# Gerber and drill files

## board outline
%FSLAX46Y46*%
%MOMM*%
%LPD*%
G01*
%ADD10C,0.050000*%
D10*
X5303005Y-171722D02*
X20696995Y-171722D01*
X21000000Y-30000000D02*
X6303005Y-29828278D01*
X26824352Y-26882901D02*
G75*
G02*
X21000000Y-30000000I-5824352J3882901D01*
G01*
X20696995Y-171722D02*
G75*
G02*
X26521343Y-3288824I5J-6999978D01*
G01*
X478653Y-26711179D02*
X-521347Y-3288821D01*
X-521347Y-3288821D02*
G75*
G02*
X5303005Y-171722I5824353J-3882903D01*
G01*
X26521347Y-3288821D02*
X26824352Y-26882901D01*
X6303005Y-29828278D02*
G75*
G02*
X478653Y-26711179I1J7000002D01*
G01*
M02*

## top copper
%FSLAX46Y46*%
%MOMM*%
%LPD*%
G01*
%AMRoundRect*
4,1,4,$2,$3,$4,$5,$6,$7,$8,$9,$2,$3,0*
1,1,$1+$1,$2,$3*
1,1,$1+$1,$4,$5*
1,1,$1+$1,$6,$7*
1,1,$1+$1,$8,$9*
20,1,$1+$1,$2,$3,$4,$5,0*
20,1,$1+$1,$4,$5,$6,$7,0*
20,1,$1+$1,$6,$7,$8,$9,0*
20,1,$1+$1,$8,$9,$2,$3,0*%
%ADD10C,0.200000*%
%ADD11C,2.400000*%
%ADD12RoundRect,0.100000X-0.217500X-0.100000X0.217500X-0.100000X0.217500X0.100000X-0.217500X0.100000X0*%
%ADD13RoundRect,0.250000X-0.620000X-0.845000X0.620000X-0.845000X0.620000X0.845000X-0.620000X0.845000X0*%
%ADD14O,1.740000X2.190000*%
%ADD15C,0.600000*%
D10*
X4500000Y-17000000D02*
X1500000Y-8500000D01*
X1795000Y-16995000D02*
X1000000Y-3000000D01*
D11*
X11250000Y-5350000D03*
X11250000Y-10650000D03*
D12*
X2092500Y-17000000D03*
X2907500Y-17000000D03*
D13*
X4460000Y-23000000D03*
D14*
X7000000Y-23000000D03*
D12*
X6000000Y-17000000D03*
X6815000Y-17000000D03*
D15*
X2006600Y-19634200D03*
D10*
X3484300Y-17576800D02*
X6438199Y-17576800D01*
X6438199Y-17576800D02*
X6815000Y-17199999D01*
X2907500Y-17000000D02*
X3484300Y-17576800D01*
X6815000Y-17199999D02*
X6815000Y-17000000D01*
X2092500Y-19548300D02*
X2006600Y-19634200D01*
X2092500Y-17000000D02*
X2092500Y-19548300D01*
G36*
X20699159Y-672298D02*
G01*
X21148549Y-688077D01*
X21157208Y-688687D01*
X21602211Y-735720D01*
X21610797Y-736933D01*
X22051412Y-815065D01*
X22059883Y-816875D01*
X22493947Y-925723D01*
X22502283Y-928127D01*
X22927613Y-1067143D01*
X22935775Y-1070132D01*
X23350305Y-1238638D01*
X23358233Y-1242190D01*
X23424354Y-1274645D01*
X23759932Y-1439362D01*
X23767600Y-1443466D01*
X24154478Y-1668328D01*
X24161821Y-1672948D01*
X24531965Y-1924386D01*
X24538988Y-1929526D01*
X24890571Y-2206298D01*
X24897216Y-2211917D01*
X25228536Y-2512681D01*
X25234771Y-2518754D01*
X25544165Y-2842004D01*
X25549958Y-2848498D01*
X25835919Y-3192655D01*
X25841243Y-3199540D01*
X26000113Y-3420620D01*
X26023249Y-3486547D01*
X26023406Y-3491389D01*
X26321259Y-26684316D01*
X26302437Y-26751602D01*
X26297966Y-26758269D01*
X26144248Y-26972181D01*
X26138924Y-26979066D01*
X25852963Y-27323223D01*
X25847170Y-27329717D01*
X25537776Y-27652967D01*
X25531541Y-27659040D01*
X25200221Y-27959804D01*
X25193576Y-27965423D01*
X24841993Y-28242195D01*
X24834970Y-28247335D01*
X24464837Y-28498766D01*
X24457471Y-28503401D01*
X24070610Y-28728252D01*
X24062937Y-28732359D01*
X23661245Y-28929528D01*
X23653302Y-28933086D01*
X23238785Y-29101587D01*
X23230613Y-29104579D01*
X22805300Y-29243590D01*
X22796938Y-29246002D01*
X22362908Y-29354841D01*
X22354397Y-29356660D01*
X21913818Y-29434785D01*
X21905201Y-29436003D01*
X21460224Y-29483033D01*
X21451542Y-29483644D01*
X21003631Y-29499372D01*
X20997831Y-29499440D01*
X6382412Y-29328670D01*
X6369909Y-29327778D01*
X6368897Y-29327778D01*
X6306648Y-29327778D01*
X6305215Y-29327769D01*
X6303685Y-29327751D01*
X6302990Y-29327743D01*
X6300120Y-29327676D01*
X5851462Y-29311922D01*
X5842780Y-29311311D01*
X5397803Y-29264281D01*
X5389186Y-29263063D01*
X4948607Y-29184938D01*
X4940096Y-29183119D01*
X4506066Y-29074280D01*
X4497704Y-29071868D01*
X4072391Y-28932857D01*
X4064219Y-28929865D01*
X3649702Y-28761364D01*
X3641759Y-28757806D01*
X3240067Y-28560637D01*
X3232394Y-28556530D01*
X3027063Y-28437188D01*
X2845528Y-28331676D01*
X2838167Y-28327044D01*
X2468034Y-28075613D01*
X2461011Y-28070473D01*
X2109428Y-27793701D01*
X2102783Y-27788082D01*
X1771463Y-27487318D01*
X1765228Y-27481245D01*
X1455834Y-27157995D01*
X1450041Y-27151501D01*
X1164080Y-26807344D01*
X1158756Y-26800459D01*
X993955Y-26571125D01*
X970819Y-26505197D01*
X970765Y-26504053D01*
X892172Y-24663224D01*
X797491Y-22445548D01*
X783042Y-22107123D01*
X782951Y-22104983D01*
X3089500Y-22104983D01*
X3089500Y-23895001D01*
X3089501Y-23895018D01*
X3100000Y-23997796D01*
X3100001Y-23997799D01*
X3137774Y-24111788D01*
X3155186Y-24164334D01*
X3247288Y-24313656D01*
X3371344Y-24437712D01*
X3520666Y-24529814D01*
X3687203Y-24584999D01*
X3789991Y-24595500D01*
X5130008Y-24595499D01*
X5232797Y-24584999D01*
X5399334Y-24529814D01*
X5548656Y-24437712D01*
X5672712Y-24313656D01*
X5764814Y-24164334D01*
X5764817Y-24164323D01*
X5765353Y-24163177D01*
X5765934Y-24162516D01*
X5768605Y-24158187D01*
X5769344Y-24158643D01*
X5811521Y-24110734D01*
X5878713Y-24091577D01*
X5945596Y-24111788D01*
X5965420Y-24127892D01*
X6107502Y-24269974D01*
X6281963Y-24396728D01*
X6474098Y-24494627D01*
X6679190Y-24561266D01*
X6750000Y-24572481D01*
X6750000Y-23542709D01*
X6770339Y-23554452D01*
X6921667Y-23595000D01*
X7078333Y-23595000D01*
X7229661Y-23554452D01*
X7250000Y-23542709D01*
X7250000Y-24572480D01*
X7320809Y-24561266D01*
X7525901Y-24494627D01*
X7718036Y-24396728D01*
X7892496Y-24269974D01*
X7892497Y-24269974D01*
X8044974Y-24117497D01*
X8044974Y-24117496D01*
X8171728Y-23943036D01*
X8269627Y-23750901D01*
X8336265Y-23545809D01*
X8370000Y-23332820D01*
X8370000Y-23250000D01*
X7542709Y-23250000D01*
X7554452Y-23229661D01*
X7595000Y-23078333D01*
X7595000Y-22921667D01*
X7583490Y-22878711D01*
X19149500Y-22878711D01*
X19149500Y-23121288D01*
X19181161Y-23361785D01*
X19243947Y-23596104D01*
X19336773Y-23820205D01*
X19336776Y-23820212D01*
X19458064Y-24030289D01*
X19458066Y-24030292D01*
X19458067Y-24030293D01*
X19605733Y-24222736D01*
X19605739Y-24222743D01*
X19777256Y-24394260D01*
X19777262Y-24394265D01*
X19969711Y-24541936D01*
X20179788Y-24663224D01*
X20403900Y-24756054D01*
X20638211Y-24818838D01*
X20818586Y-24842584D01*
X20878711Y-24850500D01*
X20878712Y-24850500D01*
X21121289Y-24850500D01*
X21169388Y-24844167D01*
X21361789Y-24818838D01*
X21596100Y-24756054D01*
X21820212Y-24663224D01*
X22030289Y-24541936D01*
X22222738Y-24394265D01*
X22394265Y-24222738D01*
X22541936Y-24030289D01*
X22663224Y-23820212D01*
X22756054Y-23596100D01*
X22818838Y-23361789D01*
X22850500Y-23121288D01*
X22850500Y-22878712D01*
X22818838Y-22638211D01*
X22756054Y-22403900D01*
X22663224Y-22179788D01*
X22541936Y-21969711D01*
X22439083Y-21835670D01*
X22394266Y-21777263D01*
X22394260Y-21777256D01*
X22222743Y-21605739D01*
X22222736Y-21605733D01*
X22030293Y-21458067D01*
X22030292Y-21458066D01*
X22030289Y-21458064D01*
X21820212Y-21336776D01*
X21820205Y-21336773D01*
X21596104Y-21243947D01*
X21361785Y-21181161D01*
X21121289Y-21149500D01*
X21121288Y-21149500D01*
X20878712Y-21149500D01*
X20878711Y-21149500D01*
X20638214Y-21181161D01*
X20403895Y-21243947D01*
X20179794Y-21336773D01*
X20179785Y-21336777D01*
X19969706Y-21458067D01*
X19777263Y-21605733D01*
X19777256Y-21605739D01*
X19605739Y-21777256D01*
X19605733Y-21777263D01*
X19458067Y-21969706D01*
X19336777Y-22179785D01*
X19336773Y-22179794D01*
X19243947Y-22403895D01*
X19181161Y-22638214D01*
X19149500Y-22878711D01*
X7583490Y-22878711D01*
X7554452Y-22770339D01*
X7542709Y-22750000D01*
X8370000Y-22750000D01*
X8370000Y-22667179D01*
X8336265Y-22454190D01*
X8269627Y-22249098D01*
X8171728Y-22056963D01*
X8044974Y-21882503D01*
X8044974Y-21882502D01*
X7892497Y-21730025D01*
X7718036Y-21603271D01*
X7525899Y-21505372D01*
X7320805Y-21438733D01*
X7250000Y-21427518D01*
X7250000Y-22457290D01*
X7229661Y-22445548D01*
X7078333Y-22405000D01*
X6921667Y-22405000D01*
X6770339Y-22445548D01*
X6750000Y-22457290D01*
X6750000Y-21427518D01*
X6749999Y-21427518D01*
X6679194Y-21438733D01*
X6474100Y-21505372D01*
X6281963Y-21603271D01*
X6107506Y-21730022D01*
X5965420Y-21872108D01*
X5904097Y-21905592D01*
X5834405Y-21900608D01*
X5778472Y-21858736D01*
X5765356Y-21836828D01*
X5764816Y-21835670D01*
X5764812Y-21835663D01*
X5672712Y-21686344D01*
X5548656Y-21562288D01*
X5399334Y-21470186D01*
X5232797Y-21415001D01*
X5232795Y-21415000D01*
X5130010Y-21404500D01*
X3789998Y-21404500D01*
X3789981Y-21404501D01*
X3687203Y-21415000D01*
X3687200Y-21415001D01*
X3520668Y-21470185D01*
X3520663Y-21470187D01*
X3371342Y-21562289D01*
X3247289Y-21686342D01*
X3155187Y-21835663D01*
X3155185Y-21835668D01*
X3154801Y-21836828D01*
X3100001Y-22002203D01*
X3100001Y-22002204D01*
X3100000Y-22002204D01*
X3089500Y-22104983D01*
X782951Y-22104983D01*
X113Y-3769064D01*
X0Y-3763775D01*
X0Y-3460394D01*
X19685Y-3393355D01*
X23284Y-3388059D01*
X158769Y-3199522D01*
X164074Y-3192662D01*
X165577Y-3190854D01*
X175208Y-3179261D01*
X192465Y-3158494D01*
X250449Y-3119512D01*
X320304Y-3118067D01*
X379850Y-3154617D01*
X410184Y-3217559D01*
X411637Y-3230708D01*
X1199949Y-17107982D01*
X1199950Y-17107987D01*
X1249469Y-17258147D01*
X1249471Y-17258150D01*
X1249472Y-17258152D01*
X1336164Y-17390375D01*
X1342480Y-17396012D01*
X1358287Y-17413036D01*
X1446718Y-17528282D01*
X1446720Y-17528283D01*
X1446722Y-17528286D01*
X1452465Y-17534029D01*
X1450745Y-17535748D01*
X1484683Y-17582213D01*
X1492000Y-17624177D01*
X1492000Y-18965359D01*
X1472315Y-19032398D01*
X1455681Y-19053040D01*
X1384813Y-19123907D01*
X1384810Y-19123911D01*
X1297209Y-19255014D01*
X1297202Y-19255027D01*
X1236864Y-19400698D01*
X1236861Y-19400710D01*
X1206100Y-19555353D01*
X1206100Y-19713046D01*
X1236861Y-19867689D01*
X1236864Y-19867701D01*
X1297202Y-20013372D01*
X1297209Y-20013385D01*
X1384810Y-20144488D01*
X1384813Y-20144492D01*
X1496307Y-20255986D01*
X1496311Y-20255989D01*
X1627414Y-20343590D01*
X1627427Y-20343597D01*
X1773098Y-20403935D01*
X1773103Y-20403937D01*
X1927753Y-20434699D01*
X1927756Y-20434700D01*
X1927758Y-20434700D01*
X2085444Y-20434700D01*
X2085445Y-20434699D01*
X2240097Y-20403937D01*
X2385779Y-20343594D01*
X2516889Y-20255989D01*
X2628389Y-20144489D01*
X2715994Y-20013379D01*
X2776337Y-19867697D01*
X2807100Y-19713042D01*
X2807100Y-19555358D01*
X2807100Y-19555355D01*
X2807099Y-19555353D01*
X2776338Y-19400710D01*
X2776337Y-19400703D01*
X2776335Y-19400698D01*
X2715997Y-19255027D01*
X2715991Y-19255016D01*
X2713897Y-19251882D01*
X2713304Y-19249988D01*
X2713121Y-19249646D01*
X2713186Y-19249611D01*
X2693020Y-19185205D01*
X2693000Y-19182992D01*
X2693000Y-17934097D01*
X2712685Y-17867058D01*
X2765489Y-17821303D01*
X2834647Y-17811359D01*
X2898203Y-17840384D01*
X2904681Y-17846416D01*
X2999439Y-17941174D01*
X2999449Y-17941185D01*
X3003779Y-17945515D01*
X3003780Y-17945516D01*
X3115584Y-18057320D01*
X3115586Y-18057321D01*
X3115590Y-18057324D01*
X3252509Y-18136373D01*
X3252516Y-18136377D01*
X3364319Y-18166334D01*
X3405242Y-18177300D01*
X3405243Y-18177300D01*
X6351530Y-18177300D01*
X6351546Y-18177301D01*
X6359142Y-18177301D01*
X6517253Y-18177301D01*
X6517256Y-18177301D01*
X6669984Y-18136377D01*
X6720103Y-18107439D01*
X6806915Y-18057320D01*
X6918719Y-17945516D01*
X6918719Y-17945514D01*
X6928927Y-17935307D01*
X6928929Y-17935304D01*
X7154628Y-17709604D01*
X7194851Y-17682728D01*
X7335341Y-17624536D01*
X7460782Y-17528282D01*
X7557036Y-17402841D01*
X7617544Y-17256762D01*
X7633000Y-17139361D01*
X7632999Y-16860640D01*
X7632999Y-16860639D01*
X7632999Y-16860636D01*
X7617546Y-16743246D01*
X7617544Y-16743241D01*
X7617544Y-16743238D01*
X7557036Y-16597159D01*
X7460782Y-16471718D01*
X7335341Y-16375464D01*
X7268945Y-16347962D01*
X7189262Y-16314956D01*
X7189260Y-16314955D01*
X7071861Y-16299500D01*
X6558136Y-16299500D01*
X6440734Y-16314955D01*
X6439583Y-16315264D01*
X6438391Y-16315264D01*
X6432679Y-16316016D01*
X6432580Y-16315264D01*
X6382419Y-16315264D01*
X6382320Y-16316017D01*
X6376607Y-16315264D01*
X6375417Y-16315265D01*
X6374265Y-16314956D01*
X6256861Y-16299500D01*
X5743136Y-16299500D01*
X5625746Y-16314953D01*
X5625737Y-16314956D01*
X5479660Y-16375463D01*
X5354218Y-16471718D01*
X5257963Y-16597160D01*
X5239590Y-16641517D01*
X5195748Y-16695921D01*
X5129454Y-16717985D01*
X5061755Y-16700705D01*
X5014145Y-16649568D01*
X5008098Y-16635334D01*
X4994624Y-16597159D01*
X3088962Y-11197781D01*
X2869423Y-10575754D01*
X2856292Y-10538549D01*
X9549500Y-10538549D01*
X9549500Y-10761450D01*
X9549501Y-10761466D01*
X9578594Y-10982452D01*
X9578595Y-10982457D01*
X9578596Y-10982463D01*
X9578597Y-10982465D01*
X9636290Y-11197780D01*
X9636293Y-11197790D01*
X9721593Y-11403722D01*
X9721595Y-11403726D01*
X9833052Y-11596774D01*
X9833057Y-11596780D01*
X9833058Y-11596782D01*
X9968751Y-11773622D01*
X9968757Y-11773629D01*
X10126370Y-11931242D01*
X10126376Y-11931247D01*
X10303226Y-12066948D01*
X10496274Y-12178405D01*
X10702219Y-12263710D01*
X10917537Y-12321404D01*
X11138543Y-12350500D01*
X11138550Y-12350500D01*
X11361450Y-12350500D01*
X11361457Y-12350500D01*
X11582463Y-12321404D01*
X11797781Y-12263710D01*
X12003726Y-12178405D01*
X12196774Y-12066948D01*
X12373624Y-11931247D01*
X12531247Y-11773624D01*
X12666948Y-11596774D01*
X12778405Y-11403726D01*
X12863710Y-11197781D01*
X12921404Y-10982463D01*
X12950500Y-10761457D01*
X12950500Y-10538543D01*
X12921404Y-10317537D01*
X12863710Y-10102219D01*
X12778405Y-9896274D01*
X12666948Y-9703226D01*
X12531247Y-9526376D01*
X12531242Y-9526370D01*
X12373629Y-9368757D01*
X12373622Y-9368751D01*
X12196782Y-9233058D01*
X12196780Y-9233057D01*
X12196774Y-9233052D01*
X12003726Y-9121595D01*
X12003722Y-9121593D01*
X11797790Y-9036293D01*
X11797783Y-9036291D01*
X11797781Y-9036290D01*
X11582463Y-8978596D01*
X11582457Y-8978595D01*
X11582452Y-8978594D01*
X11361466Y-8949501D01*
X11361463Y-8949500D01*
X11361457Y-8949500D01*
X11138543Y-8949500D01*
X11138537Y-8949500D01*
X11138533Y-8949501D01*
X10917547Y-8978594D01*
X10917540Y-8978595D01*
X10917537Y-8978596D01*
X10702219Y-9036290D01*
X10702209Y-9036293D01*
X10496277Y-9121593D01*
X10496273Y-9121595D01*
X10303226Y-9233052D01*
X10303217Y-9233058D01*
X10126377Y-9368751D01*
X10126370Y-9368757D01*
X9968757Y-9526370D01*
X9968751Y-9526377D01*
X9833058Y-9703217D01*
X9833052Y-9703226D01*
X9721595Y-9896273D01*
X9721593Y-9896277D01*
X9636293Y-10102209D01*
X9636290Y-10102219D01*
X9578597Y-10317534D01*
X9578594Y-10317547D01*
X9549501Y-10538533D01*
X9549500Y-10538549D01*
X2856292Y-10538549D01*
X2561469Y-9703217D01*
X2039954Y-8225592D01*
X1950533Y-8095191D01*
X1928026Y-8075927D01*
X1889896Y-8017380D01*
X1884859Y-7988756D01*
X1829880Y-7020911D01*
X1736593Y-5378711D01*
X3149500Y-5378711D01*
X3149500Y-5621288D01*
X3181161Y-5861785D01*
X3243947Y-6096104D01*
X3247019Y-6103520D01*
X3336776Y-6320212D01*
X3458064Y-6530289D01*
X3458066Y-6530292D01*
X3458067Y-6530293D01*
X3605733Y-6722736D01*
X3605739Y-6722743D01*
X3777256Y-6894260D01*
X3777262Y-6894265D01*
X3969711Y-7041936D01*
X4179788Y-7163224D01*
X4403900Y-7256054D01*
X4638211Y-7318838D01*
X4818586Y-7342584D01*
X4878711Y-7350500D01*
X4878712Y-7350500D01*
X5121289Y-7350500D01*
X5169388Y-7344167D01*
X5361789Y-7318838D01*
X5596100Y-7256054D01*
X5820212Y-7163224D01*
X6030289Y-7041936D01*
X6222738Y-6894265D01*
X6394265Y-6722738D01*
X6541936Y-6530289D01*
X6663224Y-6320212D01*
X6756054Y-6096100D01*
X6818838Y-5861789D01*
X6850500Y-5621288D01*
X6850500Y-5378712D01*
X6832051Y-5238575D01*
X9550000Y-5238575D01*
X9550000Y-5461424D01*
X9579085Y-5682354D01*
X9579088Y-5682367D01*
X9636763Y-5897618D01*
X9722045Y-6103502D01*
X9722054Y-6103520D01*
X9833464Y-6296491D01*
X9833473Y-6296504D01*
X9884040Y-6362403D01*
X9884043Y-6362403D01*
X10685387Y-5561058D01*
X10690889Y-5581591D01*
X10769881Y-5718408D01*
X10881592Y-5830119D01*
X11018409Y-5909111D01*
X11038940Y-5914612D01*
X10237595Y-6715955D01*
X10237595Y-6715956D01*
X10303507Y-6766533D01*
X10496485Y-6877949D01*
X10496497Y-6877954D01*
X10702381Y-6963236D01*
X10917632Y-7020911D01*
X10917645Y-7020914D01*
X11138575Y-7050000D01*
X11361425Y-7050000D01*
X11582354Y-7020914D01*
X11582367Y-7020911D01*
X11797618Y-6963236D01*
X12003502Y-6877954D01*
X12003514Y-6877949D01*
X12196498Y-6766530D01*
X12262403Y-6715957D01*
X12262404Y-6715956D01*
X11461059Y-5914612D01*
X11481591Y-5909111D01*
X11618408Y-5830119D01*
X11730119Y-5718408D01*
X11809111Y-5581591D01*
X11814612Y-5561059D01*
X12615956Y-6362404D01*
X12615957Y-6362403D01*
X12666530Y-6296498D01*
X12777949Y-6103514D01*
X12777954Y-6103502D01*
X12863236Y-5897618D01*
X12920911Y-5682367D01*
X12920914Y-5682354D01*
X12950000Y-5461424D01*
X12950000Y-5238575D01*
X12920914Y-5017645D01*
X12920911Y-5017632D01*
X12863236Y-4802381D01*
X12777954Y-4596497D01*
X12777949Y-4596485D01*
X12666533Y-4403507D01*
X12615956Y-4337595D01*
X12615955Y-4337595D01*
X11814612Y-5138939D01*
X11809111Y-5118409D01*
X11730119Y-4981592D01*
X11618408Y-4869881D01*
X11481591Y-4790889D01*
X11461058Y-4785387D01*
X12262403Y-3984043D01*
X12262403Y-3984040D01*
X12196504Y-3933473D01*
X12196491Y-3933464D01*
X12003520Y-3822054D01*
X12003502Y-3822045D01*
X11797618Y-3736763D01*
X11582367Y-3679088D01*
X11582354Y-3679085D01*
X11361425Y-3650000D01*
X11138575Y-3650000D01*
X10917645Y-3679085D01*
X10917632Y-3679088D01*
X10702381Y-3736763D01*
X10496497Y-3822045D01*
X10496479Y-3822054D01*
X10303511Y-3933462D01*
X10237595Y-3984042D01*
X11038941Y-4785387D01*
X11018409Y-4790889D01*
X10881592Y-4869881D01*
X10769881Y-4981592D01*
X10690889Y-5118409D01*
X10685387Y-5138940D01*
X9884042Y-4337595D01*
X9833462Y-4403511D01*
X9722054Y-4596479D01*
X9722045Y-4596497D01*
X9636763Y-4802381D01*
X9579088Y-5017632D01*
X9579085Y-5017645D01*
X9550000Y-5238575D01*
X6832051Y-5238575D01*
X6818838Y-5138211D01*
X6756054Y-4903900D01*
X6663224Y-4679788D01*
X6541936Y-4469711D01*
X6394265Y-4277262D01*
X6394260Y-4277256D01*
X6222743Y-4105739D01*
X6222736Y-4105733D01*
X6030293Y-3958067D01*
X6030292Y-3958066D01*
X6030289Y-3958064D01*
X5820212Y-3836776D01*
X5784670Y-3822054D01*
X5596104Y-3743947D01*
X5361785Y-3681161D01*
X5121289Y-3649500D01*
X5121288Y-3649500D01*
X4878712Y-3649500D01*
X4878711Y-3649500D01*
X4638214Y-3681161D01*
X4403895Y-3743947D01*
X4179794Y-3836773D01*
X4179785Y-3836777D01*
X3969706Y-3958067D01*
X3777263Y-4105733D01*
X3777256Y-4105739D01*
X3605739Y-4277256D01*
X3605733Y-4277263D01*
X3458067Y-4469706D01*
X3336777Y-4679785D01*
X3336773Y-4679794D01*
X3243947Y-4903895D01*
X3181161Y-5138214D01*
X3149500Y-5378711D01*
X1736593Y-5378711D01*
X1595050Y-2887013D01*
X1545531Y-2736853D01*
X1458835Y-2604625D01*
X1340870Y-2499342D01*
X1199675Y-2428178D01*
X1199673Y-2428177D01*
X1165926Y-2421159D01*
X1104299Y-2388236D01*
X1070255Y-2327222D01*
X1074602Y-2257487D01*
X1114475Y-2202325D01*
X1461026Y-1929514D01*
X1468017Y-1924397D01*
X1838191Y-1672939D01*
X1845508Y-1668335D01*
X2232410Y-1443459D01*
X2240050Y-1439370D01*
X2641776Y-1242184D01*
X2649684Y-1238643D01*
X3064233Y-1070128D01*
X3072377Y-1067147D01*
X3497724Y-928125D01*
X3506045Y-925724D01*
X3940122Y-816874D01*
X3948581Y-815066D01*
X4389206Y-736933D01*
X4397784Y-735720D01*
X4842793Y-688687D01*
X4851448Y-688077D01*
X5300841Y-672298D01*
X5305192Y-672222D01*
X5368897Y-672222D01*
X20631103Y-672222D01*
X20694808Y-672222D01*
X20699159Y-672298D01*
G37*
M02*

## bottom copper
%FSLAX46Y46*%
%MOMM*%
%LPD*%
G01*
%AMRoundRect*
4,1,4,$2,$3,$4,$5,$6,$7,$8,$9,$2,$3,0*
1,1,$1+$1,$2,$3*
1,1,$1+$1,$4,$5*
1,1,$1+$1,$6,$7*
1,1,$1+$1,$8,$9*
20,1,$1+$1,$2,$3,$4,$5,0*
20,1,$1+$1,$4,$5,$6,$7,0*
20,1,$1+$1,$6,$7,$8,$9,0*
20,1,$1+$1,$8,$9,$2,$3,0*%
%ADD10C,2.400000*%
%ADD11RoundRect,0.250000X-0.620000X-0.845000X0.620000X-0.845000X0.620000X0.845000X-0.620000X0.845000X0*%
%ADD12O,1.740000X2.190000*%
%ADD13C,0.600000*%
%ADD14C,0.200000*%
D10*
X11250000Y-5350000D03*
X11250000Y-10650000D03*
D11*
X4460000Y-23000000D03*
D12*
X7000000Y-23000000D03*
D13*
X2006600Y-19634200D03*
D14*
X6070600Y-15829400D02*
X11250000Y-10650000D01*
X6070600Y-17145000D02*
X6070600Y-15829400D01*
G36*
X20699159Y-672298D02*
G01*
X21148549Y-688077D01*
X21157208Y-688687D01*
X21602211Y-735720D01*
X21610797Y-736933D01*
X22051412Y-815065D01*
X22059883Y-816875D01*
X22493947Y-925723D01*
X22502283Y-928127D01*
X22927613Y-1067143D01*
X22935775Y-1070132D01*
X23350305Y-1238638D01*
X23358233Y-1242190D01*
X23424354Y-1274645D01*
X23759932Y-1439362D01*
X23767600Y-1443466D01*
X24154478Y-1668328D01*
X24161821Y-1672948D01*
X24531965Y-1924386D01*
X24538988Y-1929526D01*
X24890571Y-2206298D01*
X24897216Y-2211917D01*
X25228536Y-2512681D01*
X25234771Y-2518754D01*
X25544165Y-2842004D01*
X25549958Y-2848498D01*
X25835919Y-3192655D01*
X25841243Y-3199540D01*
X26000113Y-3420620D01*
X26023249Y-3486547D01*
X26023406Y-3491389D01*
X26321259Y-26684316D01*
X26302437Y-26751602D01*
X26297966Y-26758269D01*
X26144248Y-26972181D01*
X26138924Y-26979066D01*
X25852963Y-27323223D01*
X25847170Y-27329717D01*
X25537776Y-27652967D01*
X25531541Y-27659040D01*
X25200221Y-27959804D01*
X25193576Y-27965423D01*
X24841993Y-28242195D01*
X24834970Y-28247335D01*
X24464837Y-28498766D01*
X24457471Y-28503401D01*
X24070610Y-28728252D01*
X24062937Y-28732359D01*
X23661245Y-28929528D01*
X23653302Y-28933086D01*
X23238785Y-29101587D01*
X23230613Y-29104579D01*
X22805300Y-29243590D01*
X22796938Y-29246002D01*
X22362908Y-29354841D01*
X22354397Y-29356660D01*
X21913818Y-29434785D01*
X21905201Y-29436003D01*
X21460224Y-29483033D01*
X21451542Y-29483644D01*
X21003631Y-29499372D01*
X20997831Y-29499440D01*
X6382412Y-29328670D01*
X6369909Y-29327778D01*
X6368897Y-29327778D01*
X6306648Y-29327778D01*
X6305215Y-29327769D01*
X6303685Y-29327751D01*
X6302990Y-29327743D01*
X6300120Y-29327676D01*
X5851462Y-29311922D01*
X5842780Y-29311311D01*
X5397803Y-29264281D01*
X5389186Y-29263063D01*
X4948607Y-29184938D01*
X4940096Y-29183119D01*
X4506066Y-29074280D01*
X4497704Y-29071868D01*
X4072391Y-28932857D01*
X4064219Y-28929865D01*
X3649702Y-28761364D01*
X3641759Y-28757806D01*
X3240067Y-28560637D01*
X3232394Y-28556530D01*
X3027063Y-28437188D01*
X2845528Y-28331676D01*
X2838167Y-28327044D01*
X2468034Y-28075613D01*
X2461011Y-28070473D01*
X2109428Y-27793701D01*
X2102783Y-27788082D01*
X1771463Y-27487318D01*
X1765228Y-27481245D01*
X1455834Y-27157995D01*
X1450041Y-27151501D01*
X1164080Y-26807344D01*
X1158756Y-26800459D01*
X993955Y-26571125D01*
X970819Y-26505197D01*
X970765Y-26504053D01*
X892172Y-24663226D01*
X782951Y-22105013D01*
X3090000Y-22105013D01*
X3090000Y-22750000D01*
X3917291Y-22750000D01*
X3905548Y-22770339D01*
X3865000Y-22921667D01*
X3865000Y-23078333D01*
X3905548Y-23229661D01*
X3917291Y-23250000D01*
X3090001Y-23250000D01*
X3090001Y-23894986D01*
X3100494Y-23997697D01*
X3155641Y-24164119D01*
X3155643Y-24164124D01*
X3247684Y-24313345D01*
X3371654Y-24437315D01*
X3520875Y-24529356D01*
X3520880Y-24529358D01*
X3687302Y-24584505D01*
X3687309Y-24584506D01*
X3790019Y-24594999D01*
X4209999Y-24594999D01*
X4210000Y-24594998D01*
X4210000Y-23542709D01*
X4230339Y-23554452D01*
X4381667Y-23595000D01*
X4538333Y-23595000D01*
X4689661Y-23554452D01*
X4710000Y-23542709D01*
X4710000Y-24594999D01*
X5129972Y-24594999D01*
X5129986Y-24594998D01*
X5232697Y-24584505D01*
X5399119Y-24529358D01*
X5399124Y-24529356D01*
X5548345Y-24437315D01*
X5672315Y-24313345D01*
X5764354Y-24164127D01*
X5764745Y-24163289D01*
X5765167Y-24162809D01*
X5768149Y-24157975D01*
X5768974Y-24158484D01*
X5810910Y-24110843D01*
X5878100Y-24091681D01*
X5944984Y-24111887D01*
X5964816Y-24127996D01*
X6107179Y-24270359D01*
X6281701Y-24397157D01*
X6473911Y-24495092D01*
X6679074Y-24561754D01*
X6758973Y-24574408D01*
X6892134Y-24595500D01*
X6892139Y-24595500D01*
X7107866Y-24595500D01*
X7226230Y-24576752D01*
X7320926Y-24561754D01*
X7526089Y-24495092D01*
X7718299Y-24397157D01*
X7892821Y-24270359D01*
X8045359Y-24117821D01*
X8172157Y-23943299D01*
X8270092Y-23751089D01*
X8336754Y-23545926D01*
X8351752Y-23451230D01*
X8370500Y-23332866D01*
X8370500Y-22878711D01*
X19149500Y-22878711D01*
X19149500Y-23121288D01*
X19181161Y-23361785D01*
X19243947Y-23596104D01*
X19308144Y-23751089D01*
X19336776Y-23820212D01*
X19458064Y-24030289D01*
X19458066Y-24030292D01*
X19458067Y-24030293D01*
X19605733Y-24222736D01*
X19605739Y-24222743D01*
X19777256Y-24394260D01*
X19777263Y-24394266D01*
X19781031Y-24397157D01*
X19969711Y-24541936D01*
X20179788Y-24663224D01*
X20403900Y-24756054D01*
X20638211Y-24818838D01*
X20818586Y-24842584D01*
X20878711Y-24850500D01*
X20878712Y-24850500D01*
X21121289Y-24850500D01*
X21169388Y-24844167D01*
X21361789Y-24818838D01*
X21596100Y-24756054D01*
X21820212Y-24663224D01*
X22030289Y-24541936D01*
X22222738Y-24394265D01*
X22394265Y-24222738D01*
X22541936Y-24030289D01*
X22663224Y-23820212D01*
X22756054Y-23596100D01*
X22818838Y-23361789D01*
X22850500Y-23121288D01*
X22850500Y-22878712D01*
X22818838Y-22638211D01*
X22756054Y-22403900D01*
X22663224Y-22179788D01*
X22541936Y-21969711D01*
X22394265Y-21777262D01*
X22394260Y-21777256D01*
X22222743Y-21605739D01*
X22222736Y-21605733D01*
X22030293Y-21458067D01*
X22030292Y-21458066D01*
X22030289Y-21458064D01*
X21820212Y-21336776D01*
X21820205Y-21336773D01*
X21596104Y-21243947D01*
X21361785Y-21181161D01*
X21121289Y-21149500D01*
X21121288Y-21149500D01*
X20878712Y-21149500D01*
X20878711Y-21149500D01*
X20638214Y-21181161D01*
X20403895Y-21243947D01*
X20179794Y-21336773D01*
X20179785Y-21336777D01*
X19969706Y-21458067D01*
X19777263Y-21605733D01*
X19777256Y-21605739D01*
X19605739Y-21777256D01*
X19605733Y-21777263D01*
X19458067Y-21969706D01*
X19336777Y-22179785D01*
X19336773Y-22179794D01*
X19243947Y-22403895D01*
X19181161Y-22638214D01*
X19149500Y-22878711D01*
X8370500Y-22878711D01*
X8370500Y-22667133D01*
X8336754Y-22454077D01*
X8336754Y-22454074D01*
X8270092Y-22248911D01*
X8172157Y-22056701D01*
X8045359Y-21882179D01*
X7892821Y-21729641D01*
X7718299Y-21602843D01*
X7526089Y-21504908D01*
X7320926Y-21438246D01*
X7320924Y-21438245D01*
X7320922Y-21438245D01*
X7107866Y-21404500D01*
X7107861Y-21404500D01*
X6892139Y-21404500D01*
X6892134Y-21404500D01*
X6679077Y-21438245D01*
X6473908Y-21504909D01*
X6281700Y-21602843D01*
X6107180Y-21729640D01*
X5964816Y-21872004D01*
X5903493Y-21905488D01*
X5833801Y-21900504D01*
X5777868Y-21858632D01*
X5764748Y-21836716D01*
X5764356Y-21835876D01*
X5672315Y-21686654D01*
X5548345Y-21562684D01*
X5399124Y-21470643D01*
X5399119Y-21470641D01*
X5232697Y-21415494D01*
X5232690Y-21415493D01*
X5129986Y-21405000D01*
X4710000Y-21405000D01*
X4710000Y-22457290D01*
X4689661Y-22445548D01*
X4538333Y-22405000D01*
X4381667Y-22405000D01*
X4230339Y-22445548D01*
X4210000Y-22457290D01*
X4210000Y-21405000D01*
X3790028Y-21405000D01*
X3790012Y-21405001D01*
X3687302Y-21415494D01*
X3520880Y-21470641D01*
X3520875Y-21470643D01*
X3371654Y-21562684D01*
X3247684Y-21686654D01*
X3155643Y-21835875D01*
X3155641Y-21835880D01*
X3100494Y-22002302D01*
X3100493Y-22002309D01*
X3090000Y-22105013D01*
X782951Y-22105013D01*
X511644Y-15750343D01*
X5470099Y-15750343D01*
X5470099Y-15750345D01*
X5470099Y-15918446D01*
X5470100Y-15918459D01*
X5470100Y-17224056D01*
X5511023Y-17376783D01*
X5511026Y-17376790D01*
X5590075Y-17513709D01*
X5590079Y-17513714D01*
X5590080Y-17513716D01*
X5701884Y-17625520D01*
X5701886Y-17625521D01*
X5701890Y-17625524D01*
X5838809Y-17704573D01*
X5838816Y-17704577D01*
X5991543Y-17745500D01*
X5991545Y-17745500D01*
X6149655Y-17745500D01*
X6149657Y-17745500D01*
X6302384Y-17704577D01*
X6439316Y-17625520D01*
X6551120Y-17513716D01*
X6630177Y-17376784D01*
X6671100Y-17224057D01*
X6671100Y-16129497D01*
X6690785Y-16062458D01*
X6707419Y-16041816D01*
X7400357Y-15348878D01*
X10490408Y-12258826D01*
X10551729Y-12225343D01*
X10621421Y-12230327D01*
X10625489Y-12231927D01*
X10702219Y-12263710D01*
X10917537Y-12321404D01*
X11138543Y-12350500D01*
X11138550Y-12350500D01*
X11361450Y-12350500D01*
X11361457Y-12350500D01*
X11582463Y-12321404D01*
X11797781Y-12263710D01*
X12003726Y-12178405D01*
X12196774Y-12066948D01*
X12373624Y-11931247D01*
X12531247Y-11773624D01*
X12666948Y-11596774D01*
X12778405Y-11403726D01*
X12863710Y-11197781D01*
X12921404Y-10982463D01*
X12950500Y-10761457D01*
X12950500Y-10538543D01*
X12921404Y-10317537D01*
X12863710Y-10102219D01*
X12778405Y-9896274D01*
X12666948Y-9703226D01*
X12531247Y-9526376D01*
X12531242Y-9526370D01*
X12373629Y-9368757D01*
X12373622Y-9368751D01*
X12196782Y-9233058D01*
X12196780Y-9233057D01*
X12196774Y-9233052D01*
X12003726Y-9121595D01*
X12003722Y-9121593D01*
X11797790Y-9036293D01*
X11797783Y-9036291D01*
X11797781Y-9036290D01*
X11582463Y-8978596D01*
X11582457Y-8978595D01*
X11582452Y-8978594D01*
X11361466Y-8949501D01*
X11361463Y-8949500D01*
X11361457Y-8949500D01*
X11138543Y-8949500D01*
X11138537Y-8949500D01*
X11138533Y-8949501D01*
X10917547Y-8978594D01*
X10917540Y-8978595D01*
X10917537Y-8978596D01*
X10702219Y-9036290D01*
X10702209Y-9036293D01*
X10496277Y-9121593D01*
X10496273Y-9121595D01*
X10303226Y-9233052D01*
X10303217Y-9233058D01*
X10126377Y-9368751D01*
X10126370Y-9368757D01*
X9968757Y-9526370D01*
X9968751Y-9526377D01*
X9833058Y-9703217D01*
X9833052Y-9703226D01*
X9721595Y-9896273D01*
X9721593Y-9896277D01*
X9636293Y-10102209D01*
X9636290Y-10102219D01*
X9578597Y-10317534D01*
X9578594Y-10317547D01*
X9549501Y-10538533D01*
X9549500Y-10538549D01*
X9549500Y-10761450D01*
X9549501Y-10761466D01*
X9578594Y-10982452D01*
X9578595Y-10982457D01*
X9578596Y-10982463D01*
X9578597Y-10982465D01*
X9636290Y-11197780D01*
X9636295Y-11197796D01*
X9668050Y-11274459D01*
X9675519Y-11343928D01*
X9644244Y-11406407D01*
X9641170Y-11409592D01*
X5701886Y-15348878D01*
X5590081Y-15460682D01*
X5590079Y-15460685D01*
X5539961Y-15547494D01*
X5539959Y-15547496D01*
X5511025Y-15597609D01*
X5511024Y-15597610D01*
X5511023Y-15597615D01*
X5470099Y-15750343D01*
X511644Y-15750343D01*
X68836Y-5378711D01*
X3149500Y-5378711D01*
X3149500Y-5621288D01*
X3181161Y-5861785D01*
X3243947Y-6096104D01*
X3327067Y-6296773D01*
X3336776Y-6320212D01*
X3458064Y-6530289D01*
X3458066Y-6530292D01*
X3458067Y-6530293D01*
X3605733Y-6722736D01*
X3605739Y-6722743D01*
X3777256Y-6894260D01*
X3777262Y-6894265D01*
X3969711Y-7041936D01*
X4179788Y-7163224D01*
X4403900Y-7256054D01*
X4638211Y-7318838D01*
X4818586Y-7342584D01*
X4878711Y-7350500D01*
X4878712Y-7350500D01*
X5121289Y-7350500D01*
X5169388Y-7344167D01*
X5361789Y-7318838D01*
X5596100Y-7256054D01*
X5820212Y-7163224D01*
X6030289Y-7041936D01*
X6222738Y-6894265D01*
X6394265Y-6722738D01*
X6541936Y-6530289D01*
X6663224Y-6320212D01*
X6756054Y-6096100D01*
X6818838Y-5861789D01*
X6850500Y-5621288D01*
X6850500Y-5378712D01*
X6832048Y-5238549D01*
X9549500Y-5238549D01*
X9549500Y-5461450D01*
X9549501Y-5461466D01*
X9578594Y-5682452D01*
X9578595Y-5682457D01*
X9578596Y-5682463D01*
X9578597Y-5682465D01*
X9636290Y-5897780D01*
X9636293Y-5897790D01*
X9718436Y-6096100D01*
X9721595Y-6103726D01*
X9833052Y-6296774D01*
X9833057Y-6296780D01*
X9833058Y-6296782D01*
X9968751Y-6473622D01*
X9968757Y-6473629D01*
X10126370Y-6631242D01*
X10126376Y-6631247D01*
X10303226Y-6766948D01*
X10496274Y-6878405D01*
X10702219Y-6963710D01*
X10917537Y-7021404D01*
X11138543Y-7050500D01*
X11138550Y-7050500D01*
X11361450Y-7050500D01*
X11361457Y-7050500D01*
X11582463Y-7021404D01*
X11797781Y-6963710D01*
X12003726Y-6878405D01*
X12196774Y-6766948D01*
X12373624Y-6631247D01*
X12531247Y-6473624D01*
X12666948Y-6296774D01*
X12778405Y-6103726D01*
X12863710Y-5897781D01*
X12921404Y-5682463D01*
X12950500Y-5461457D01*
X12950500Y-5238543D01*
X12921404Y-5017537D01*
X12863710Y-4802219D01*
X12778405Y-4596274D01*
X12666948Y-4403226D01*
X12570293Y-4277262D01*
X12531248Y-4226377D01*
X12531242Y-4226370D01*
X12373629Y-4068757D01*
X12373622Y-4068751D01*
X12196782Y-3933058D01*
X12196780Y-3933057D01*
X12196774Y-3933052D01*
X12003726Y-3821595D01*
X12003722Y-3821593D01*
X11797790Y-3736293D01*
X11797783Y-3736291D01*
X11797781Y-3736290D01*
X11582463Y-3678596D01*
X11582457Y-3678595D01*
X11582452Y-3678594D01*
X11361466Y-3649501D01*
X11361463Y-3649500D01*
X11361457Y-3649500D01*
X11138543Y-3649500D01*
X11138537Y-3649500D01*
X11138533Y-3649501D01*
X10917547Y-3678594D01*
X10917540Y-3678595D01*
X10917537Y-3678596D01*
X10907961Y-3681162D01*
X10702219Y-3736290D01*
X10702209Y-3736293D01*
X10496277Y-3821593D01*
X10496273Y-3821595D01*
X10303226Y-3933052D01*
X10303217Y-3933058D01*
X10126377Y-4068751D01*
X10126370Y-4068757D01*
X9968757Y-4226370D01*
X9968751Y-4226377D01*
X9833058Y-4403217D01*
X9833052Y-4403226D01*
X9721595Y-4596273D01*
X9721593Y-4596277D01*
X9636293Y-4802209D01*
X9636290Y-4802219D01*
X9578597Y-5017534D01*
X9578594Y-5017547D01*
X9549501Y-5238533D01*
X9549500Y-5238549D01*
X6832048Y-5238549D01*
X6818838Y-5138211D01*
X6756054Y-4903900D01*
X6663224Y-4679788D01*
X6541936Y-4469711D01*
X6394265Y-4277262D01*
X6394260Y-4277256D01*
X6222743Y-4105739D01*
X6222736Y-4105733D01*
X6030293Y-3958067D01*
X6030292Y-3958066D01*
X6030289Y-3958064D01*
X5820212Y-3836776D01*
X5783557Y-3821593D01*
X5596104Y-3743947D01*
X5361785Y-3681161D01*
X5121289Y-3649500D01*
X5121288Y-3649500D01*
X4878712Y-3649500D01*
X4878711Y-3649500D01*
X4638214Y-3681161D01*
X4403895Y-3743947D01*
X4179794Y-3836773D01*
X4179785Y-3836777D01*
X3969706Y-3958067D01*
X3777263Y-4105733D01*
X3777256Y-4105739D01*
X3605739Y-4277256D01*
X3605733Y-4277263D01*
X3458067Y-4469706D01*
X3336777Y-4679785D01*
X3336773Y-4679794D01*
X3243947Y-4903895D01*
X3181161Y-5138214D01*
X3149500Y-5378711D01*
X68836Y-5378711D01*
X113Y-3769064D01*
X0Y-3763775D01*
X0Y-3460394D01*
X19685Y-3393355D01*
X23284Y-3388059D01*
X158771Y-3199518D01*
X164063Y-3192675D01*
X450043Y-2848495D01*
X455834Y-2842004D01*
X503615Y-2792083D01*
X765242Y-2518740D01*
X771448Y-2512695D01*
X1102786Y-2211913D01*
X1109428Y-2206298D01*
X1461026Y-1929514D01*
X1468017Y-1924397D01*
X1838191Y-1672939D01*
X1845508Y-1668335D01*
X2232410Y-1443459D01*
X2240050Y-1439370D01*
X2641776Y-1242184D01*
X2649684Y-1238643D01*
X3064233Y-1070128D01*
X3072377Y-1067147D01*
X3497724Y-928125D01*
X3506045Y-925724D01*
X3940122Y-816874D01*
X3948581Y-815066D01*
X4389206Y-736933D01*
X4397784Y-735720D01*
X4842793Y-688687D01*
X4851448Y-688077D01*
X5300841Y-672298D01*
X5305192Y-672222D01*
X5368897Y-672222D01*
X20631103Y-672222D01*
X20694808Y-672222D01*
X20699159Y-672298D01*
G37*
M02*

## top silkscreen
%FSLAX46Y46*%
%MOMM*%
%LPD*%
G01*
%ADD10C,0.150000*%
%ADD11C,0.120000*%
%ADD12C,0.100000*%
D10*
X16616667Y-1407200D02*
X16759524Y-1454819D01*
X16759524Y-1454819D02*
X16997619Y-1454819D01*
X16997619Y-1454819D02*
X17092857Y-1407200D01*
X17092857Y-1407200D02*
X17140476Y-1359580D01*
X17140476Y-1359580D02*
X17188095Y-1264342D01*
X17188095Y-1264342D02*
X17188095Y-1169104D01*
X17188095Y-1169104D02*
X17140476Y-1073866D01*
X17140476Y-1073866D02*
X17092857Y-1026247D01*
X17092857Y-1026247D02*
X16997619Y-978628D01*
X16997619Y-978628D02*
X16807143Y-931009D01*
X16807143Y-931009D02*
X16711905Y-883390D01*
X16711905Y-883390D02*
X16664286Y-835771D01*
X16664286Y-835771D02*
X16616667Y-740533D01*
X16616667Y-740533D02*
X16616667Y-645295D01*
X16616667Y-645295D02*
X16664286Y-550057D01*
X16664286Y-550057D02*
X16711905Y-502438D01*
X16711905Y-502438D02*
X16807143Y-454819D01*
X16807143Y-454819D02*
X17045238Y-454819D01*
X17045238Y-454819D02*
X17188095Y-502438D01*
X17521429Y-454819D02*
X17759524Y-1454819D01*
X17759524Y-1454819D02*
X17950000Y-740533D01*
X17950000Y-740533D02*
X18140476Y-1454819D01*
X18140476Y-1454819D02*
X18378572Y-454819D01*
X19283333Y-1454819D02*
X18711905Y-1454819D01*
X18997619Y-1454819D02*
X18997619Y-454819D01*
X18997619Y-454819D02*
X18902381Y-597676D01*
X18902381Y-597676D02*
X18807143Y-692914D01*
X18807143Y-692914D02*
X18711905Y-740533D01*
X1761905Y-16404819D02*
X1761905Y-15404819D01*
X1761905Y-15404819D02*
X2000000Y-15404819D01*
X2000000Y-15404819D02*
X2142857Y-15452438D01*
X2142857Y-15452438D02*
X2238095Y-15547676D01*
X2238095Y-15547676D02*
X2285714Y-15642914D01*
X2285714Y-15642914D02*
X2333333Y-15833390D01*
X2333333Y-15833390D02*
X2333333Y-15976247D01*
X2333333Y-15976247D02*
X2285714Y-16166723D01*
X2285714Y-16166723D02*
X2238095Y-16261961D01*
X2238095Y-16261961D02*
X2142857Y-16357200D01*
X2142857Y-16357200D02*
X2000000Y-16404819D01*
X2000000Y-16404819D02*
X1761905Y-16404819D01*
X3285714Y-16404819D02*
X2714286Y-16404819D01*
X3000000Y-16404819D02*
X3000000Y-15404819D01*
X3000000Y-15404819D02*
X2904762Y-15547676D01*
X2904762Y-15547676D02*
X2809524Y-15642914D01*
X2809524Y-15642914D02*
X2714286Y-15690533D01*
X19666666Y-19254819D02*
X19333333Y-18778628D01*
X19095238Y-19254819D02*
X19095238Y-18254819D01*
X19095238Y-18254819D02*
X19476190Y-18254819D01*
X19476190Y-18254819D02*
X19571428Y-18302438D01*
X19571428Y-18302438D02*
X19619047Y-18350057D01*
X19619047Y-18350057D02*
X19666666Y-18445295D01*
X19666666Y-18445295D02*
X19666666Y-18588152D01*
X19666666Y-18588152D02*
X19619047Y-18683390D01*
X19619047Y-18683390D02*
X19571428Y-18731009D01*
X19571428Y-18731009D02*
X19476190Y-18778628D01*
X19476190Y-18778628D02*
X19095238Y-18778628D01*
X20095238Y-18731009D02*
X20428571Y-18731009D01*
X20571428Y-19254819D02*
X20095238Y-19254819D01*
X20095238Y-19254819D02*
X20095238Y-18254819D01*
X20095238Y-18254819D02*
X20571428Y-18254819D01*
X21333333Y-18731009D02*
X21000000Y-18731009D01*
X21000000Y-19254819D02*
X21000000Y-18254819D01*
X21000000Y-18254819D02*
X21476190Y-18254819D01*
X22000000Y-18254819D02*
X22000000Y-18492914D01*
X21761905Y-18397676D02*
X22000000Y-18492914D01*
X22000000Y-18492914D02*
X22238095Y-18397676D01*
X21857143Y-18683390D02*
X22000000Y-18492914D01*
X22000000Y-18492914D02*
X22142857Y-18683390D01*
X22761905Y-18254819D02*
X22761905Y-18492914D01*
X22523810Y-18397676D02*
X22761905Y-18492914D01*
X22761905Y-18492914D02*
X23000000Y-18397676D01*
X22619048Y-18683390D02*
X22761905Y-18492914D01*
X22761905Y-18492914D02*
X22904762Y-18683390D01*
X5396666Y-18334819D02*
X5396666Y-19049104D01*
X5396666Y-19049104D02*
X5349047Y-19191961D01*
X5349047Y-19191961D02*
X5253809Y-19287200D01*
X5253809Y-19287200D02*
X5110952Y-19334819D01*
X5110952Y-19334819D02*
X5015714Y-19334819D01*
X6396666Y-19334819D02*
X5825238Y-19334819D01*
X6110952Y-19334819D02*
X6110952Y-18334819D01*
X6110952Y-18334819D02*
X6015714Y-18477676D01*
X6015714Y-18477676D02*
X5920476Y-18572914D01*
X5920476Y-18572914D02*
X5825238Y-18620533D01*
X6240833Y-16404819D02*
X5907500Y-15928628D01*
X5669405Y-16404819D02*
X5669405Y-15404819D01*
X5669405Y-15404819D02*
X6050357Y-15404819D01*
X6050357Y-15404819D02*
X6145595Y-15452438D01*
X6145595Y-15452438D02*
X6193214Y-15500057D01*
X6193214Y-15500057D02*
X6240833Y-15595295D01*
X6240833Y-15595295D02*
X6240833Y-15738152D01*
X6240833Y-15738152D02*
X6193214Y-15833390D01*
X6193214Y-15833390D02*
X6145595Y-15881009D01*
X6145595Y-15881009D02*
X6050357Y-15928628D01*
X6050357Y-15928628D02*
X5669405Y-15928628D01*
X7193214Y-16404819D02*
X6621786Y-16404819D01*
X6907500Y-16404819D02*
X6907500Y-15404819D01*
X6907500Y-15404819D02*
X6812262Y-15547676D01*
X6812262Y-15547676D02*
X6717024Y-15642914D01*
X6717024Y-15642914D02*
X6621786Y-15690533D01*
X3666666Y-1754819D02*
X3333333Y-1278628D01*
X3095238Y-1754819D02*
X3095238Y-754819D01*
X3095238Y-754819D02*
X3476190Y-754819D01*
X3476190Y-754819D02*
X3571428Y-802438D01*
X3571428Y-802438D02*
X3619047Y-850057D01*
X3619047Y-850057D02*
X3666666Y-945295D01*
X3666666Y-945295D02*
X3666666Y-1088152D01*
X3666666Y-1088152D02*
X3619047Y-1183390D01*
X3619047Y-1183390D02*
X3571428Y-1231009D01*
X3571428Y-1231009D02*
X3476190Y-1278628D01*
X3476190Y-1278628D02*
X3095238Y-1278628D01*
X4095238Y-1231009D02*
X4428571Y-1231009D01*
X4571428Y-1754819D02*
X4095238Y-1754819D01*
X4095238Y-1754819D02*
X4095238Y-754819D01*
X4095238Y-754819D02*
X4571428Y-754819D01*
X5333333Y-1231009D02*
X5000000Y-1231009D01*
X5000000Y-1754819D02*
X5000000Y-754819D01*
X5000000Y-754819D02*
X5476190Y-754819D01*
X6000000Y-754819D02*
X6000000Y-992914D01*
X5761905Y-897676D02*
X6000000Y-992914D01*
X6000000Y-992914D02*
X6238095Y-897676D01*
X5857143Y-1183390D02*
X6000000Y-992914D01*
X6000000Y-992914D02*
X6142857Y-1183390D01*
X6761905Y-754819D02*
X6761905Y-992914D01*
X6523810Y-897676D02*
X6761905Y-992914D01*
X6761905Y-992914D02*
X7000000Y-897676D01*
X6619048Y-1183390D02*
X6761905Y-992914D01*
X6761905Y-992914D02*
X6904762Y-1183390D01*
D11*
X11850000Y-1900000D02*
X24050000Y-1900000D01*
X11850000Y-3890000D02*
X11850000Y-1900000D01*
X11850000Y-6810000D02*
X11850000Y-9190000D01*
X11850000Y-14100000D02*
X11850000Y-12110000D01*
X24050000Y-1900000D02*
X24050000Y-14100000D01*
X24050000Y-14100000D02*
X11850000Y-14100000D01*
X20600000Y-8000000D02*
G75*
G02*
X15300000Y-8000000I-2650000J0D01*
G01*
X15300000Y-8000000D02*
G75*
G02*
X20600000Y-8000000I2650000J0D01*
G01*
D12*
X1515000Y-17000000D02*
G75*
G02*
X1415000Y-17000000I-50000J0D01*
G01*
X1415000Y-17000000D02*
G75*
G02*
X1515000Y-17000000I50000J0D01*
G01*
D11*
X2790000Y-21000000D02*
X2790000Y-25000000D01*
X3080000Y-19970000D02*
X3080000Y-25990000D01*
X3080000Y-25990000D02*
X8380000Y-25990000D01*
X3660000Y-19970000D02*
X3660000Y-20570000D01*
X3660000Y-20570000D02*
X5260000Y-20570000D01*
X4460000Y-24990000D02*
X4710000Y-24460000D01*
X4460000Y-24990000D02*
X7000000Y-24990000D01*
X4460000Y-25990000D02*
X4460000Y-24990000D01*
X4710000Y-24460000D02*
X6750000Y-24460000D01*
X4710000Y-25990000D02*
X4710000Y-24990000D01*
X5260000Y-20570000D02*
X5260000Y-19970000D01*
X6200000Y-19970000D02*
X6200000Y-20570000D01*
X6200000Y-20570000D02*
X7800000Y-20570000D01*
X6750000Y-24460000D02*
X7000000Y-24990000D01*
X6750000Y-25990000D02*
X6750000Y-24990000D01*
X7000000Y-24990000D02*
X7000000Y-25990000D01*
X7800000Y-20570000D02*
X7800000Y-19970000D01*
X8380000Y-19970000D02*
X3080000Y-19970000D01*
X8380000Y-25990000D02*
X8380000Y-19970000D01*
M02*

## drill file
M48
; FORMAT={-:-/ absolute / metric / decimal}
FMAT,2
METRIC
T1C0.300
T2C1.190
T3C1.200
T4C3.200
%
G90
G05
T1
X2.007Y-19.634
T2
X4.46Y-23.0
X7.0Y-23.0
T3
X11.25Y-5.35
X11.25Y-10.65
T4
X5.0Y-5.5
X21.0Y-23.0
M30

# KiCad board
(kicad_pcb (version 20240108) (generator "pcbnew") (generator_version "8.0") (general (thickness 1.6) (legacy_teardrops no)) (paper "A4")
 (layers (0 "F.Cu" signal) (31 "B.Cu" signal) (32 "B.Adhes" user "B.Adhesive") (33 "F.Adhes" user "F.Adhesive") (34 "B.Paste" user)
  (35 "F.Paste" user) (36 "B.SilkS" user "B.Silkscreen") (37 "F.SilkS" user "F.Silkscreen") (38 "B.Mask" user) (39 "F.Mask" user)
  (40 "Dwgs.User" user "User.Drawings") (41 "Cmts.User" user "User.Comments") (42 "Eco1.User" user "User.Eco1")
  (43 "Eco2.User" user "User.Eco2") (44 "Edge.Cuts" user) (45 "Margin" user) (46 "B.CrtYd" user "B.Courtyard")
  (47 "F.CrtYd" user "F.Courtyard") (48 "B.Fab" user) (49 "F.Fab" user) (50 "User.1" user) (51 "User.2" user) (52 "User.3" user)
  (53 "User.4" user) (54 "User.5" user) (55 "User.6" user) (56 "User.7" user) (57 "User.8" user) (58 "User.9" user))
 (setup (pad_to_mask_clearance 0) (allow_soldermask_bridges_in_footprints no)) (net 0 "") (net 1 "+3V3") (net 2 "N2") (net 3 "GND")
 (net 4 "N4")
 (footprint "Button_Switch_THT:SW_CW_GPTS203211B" (layer "F.Cu") (at 11.25 5.35)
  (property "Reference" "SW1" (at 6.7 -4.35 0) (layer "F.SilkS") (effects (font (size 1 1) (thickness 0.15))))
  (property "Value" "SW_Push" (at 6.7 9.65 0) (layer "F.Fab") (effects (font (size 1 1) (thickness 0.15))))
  (fp_line (start 0.6 -3.45) (end 12.8 -3.45) (stroke (width 0.12) (type solid)) (layer "F.SilkS"))
  (fp_line (start 0.6 -1.46) (end 0.6 -3.45) (stroke (width 0.12) (type solid)) (layer "F.SilkS"))
  (fp_line (start 0.6 1.46) (end 0.6 3.84) (stroke (width 0.12) (type solid)) (layer "F.SilkS"))
  (fp_line (start 0.6 8.75) (end 0.6 6.76) (stroke (width 0.12) (type solid)) (layer "F.SilkS"))
  (fp_line (start 12.8 -3.45) (end 12.8 8.75) (stroke (width 0.12) (type solid)) (layer "F.SilkS"))
  (fp_line (start 12.8 8.75) (end 0.6 8.75) (stroke (width 0.12) (type solid)) (layer "F.SilkS"))
  (fp_circle (center 6.7 2.65) (end 9.35 2.65) (stroke (width 0.12) (type solid)) (fill none) (layer "F.SilkS"))
  (pad "1" thru_hole circle (at 0 0) (size 2.4 2.4) (drill 1.2) (layers "*.Cu" "*.Mask") (remove_unused_layers no) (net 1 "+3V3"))
  (pad "2" thru_hole circle (at 0 5.3) (size 2.4 2.4) (drill 1.2) (layers "*.Cu" "*.Mask") (remove_unused_layers no) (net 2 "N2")))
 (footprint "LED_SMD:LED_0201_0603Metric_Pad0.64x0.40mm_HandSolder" (layer "F.Cu") (at 2.5 17)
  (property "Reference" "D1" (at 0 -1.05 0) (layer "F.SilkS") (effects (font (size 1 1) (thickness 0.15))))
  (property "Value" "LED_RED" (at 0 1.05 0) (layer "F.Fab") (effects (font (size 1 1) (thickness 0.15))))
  (fp_circle (center -1.035 0) (end -0.985 0) (stroke (width 0.1) (type solid)) (fill none) (layer "F.SilkS"))
  (pad "" smd roundrect (at -0.4325 0) (size 0.458 0.36) (layers "F.Paste") (roundrect_rratio 0.25))
  (pad "" smd roundrect (at 0.4325 0) (size 0.458 0.36) (layers "F.Paste") (roundrect_rratio 0.25))
  (pad "1" smd roundrect (at -0.4075 0) (size 0.635 0.4) (layers "F.Cu" "F.Mask") (roundrect_rratio 0.25) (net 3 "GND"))
  (pad "2" smd roundrect (at 0.4075 0) (size 0.635 0.4) (layers "F.Cu" "F.Mask") (roundrect_rratio 0.25) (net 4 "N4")))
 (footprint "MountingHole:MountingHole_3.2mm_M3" (layer "F.Cu") (at 21 23)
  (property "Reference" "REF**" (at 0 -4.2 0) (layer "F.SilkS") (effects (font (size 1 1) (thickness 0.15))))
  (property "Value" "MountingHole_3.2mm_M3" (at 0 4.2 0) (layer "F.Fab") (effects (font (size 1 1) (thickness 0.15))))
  (pad "" np_thru_hole circle (at 0 0) (size 3.2 3.2) (drill 3.2) (layers "*.Cu" "*.Mask")))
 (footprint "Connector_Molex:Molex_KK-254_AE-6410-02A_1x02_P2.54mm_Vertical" (layer "F.Cu") (at 4.46 23)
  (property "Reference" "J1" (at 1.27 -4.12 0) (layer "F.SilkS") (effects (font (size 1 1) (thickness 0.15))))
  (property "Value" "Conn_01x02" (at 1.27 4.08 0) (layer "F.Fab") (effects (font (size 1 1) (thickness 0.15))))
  (fp_line (start -1.67 -2) (end -1.67 2) (stroke (width 0.12) (type solid)) (layer "F.SilkS"))
  (fp_line (start -1.38 -3.03) (end -1.38 2.99) (stroke (width 0.12) (type solid)) (layer "F.SilkS"))
  (fp_line (start -1.38 2.99) (end 3.92 2.99) (stroke (width 0.12) (type solid)) (layer "F.SilkS"))
  (fp_line (start -0.8 -3.03) (end -0.8 -2.43) (stroke (width 0.12) (type solid)) (layer "F.SilkS"))
  (fp_line (start -0.8 -2.43) (end 0.8 -2.43) (stroke (width 0.12) (type solid)) (layer "F.SilkS"))
  (fp_line (start 0 1.99) (end 0.25 1.46) (stroke (width 0.12) (type solid)) (layer "F.SilkS"))
  (fp_line (start 0 1.99) (end 2.54 1.99) (stroke (width 0.12) (type solid)) (layer "F.SilkS"))
  (fp_line (start 0 2.99) (end 0 1.99) (stroke (width 0.12) (type solid)) (layer "F.SilkS"))
  (fp_line (start 0.25 1.46) (end 2.29 1.46) (stroke (width 0.12) (type solid)) (layer "F.SilkS"))
  (fp_line (start 0.25 2.99) (end 0.25 1.99) (stroke (width 0.12) (type solid)) (layer "F.SilkS"))
  (fp_line (start 0.8 -2.43) (end 0.8 -3.03) (stroke (width 0.12) (type solid)) (layer "F.SilkS"))
  (fp_line (start 1.74 -3.03) (end 1.74 -2.43) (stroke (width 0.12) (type solid)) (layer "F.SilkS"))
  (fp_line (start 1.74 -2.43) (end 3.34 -2.43) (stroke (width 0.12) (type solid)) (layer "F.SilkS"))
  (fp_line (start 2.29 1.46) (end 2.54 1.99) (stroke (width 0.12) (type solid)) (layer "F.SilkS"))
  (fp_line (start 2.29 2.99) (end 2.29 1.99) (stroke (width 0.12) (type solid)) (layer "F.SilkS"))
  (fp_line (start 2.54 1.99) (end 2.54 2.99) (stroke (width 0.12) (type solid)) (layer "F.SilkS"))
  (fp_line (start 3.34 -2.43) (end 3.34 -3.03) (stroke (width 0.12) (type solid)) (layer "F.SilkS"))
  (fp_line (start 3.92 -3.03) (end -1.38 -3.03) (stroke (width 0.12) (type solid)) (layer "F.SilkS"))
  (fp_line (start 3.92 2.99) (end 3.92 -3.03) (stroke (width 0.12) (type solid)) (layer "F.SilkS"))
  (pad "1" thru_hole roundrect (at 0 0) (size 1.74 2.19) (drill 1.19) (layers "*.Cu" "*.Mask") (remove_unused_layers no)
   (roundrect_rratio 0.143678) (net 3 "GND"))
  (pad "2" thru_hole oval (at 2.54 0) (size 1.74 2.19) (drill 1.19) (layers "*.Cu" "*.Mask") (remove_unused_layers no) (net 1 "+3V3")))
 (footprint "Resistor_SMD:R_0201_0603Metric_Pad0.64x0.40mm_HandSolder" (layer "F.Cu") (at 6.4075 17)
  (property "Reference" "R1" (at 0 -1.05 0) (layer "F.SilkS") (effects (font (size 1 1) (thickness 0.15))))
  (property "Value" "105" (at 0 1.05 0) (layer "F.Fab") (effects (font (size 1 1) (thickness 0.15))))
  (pad "" smd roundrect (at -0.4325 0) (size 0.458 0.36) (layers "F.Paste") (roundrect_rratio 0.25))
  (pad "" smd roundrect (at 0.4325 0) (size 0.458 0.36) (layers "F.Paste") (roundrect_rratio 0.25))
  (pad "1" smd roundrect (at -0.4075 0) (size 0.635 0.4) (layers "F.Cu" "F.Mask") (roundrect_rratio 0.25) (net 2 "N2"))
  (pad "2" smd roundrect (at 0.4075 0) (size 0.635 0.4) (layers "F.Cu" "F.Mask") (roundrect_rratio 0.25) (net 4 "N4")))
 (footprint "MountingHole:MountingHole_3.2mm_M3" (layer "F.Cu") (at 5 5.5)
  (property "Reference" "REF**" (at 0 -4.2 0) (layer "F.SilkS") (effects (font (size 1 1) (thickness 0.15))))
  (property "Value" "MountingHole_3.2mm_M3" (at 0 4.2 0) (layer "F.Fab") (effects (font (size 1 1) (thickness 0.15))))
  (pad "" np_thru_hole circle (at 0 0) (size 3.2 3.2) (drill 3.2) (layers "*.Cu" "*.Mask")))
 (gr_line (start 4.5 17) (end 1.5 8.5) (stroke (width 0.2) (type default)) (layer "F.Cu") (net 3))
 (gr_line (start 1.795 16.995) (end 1 3) (stroke (width 0.2) (type default)) (layer "F.Cu") (net 3))
 (gr_line (start 5.303005 0.171722) (end 20.696995 0.171722) (stroke (width 0.05) (type default)) (layer "Edge.Cuts"))
 (gr_line (start 21 30) (end 6.303005 29.828278) (stroke (width 0.05) (type default)) (layer "Edge.Cuts"))
 (gr_arc (start 26.824352 26.882901) (mid 24.303005 29.171722) (end 21 30) (stroke (width 0.05) (type default)) (layer "Edge.Cuts"))
 (gr_arc (start 20.696995 0.171722) (mid 24 1) (end 26.521347 3.288821) (stroke (width 0.05) (type default)) (layer "Edge.Cuts"))
 (gr_line (start 0.478653 26.711179) (end -0.521347 3.288821) (stroke (width 0.05) (type default)) (layer "Edge.Cuts"))
 (gr_arc (start -0.521347 3.288821) (mid 2 1) (end 5.303005 0.171722) (stroke (width 0.05) (type default)) (layer "Edge.Cuts"))
 (gr_line (start 26.521347 3.288821) (end 26.824352 26.882901) (stroke (width 0.05) (type default)) (layer "Edge.Cuts"))
 (gr_arc (start 6.303005 29.828278) (mid 3 29) (end 0.478653 26.711179) (stroke (width 0.05) (type default)) (layer "Edge.Cuts"))
 (segment (start 3.4843 17.5768) (end 6.438199 17.5768) (width 0.2) (layer "F.Cu") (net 4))
 (segment (start 6.438199 17.5768) (end 6.815 17.199999) (width 0.2) (layer "F.Cu") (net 4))
 (segment (start 2.9075 17) (end 3.4843 17.5768) (width 0.2) (layer "F.Cu") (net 4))
 (segment (start 6.815 17.199999) (end 6.815 17) (width 0.2) (layer "F.Cu") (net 4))
 (segment (start 6.0706 15.8294) (end 11.25 10.65) (width 0.2) (layer "B.Cu") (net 2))
 (segment (start 6.0706 17.145) (end 6.0706 15.8294) (width 0.2) (layer "B.Cu") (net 2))
 (segment (start 2.0925 19.5483) (end 2.0066 19.6342) (width 0.2) (layer "F.Cu") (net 3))
 (segment (start 2.0925 17) (end 2.0925 19.5483) (width 0.2) (layer "F.Cu") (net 3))
 (via (at 2.0066 19.6342) (size 0.6) (drill 0.3) (layers "F.Cu" "B.Cu") (free yes) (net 3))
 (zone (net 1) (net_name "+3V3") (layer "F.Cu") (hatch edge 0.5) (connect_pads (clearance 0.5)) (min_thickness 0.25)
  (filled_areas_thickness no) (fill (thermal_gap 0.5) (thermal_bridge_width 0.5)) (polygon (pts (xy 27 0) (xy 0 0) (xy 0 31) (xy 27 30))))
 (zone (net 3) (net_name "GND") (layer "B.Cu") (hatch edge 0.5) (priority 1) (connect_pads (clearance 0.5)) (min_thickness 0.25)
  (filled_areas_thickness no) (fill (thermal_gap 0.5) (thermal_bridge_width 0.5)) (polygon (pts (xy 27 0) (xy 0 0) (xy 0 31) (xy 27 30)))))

